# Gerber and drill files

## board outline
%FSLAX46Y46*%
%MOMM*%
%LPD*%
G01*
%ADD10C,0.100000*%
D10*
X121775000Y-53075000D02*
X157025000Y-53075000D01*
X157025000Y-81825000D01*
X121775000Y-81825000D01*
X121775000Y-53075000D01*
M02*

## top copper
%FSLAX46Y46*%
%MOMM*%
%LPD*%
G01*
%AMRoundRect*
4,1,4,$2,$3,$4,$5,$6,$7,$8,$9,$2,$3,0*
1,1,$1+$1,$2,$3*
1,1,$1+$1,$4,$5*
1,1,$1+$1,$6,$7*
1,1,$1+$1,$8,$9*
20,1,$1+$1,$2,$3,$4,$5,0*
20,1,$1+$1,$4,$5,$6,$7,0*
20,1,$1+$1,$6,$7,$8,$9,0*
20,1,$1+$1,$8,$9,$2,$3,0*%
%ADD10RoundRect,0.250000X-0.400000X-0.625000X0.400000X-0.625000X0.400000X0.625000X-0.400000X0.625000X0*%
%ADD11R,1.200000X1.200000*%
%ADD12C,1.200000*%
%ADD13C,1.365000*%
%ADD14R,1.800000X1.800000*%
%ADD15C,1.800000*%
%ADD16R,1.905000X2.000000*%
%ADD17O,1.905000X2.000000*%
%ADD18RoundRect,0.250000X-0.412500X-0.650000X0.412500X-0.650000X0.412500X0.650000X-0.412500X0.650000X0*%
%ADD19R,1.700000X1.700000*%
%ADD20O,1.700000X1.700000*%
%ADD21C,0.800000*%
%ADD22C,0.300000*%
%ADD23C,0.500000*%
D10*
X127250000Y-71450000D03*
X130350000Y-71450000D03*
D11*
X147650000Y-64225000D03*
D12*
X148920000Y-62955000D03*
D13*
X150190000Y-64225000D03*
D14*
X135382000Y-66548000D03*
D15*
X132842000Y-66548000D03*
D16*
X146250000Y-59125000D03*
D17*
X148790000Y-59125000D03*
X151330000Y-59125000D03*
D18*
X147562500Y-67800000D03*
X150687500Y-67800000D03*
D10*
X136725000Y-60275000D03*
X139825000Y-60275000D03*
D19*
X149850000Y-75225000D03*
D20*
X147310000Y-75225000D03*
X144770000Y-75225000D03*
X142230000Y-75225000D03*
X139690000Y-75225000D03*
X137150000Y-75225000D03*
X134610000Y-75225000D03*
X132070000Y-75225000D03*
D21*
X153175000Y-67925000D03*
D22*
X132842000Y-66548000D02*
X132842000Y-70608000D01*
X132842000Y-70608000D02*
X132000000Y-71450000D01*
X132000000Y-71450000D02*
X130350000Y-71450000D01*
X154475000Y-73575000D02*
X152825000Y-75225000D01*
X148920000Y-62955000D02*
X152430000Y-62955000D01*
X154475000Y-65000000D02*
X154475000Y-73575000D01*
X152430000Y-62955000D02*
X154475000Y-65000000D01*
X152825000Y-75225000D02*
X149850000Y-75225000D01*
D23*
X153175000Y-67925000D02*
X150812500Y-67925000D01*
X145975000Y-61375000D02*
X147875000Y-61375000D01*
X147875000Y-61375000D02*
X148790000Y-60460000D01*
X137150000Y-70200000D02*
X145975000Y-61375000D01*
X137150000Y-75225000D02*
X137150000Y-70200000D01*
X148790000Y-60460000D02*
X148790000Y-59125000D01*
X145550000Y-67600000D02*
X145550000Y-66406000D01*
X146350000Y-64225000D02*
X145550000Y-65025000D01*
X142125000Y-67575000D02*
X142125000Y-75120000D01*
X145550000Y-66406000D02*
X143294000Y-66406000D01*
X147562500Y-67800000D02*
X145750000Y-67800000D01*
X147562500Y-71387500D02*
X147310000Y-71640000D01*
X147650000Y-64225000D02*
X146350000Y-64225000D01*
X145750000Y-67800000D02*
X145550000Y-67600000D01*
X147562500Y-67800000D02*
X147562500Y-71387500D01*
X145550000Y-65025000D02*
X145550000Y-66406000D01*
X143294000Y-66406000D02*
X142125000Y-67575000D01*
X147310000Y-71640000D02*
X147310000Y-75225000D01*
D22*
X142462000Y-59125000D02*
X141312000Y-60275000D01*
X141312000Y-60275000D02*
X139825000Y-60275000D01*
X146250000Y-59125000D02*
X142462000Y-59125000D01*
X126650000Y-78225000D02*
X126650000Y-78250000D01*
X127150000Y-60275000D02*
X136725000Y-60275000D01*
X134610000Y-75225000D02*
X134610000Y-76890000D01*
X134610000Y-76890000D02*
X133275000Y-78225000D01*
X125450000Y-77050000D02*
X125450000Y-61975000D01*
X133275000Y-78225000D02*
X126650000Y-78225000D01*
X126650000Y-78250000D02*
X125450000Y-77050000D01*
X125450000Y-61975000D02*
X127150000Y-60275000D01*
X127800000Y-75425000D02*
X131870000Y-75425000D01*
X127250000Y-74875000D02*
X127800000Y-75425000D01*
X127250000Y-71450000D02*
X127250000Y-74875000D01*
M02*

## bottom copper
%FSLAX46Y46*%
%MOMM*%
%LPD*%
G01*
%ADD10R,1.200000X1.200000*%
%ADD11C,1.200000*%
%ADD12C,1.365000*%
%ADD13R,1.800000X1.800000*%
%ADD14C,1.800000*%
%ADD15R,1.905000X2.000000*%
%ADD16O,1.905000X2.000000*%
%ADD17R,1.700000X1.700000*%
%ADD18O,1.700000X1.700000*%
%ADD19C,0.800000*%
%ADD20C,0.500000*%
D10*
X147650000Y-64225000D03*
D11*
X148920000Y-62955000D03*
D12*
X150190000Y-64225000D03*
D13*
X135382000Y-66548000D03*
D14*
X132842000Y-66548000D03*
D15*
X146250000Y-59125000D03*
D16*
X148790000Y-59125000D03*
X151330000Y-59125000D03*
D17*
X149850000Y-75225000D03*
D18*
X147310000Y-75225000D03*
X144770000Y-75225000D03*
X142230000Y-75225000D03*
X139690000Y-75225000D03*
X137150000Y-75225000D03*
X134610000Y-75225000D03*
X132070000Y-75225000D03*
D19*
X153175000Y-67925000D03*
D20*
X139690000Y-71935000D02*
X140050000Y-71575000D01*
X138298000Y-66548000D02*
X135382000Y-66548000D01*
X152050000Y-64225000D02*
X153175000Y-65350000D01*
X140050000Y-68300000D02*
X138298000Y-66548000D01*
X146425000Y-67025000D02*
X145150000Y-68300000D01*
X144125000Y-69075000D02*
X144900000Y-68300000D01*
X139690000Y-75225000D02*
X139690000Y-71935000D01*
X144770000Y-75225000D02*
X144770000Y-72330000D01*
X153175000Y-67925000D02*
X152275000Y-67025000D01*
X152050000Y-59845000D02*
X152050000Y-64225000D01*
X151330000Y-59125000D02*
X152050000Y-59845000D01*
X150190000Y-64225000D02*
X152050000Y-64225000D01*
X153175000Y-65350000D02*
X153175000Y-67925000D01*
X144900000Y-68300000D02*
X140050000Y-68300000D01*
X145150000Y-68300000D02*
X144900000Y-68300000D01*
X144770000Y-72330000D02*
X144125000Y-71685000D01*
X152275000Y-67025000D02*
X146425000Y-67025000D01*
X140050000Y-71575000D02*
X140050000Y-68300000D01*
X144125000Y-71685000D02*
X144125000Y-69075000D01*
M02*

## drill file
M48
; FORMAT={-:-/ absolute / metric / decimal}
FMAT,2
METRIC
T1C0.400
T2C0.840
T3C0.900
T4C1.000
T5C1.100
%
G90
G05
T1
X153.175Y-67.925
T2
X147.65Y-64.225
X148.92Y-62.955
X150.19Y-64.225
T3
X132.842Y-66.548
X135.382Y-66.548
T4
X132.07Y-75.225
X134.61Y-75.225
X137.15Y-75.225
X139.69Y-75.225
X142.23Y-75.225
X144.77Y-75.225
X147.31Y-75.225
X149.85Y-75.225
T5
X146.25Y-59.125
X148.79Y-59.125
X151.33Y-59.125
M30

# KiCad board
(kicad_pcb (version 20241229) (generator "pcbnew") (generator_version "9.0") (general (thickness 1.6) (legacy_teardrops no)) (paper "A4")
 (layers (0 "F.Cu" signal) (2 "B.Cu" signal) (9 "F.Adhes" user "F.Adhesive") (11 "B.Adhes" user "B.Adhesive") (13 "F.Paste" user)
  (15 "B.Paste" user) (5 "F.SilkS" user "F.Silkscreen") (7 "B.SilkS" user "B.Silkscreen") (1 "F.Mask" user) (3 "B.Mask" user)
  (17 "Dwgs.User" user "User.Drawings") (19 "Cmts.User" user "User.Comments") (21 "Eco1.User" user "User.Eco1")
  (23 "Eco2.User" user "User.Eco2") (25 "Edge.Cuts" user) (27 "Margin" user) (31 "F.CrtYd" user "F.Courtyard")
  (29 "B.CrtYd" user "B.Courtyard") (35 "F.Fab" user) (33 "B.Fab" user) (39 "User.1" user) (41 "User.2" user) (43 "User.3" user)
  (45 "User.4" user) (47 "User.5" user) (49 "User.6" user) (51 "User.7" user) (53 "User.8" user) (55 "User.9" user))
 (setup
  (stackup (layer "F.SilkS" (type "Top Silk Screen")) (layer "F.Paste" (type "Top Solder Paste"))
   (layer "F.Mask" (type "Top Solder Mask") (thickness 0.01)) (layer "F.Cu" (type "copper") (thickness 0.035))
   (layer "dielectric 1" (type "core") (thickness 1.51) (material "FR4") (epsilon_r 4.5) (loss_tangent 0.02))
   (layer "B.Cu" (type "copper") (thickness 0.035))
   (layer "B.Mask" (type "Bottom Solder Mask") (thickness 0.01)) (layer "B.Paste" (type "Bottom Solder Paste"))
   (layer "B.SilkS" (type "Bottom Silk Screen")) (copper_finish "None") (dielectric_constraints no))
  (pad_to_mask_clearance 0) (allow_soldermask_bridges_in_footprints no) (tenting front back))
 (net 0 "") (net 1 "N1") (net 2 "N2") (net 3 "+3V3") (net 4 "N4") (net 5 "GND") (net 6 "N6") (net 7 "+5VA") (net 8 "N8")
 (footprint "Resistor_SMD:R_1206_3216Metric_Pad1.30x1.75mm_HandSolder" (layer "F.Cu") (at 128.8 71.45)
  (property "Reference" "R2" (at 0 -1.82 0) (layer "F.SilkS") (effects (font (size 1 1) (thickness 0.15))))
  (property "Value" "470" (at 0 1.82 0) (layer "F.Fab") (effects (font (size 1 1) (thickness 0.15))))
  (pad "1" smd roundrect (at -1.55 0) (size 1.3 1.75) (layers "F.Cu" "F.Mask" "F.Paste") (roundrect_rratio 0.192308) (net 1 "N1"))
  (pad "2" smd roundrect (at 1.55 0) (size 1.3 1.75) (layers "F.Cu" "F.Mask" "F.Paste") (roundrect_rratio 0.192308) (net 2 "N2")))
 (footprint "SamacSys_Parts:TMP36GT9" (layer "F.Cu") (at 147.65 64.225 90)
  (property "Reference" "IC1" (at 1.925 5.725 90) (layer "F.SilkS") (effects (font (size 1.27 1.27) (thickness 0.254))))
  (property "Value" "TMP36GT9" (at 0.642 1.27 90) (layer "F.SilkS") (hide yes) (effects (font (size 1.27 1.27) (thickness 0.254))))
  (pad "1" thru_hole rect (at 0 0 90) (size 1.2 1.2) (drill 0.84) (layers "*.Cu" "*.Mask") (remove_unused_layers no) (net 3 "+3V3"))
  (pad "2" thru_hole circle (at 1.27 1.27 90) (size 1.2 1.2) (drill 0.84) (layers "*.Cu" "*.Mask") (remove_unused_layers no) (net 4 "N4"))
  (pad "3" thru_hole circle (at 0 2.54 90) (size 1.365 1.365) (drill 0.84) (layers "*.Cu" "*.Mask") (remove_unused_layers no) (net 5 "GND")))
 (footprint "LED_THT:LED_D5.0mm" (layer "F.Cu") (at 135.382 66.548 180)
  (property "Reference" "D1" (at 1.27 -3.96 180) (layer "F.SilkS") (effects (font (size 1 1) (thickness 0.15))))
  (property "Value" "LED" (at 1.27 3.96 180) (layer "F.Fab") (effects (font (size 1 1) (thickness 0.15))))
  (pad "1" thru_hole rect (at 0 0 180) (size 1.8 1.8) (drill 0.9) (layers "*.Cu" "*.Mask") (remove_unused_layers no) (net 5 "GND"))
  (pad "2" thru_hole circle (at 2.54 0 180) (size 1.8 1.8) (drill 0.9) (layers "*.Cu" "*.Mask") (remove_unused_layers no) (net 2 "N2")))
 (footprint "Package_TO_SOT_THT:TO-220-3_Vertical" (layer "F.Cu") (at 146.25 59.125)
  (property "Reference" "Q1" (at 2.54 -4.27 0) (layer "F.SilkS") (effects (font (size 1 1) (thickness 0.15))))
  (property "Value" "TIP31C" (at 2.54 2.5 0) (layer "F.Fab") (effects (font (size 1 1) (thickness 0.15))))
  (pad "1" thru_hole rect (at 0 0) (size 1.905 2) (drill 1.1) (layers "*.Cu" "*.Mask") (remove_unused_layers no) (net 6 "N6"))
  (pad "2" thru_hole oval (at 2.54 0) (size 1.905 2) (drill 1.1) (layers "*.Cu" "*.Mask") (remove_unused_layers no) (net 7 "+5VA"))
  (pad "3" thru_hole oval (at 5.08 0) (size 1.905 2) (drill 1.1) (layers "*.Cu" "*.Mask") (remove_unused_layers no) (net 5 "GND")))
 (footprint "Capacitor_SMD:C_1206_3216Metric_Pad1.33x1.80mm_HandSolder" (layer "F.Cu") (at 149.125 67.8)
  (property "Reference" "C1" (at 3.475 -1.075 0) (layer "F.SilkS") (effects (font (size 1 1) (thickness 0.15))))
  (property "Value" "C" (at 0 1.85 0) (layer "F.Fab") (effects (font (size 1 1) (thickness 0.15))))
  (pad "1" smd roundrect (at -1.5625 0) (size 1.325 1.8) (layers "F.Cu" "F.Mask" "F.Paste") (roundrect_rratio 0.188679) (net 3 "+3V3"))
  (pad "2" smd roundrect (at 1.5625 0) (size 1.325 1.8) (layers "F.Cu" "F.Mask" "F.Paste") (roundrect_rratio 0.188679) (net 5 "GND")))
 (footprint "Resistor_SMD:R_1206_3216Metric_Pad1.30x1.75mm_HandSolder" (layer "F.Cu") (at 138.275 60.275)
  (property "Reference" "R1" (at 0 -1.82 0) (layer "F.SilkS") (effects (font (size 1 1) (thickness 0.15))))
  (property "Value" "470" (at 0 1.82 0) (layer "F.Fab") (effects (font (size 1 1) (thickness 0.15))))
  (pad "1" smd roundrect (at -1.55 0) (size 1.3 1.75) (layers "F.Cu" "F.Mask" "F.Paste") (roundrect_rratio 0.192308) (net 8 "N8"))
  (pad "2" smd roundrect (at 1.55 0) (size 1.3 1.75) (layers "F.Cu" "F.Mask" "F.Paste") (roundrect_rratio 0.192308) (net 6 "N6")))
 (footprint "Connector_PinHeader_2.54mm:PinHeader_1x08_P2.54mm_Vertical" (layer "F.Cu") (at 149.85 75.225 -90)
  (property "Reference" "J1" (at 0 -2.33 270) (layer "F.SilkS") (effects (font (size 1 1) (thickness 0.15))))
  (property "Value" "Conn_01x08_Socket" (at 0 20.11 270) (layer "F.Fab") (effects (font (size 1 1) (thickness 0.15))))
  (pad "1" thru_hole rect (at 0 0 270) (size 1.7 1.7) (drill 1) (layers "*.Cu" "*.Mask") (remove_unused_layers no) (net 4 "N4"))
  (pad "2" thru_hole oval (at 0 2.54 270) (size 1.7 1.7) (drill 1) (layers "*.Cu" "*.Mask") (remove_unused_layers no) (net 3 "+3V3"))
  (pad "3" thru_hole oval (at 0 5.08 270) (size 1.7 1.7) (drill 1) (layers "*.Cu" "*.Mask") (remove_unused_layers no) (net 5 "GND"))
  (pad "4" thru_hole oval (at 0 7.62 270) (size 1.7 1.7) (drill 1) (layers "*.Cu" "*.Mask") (remove_unused_layers no) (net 3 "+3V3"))
  (pad "5" thru_hole oval (at 0 10.16 270) (size 1.7 1.7) (drill 1) (layers "*.Cu" "*.Mask") (remove_unused_layers no) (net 5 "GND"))
  (pad "6" thru_hole oval (at 0 12.7 270) (size 1.7 1.7) (drill 1) (layers "*.Cu" "*.Mask") (remove_unused_layers no) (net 7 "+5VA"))
  (pad "7" thru_hole oval (at 0 15.24 270) (size 1.7 1.7) (drill 1) (layers "*.Cu" "*.Mask") (remove_unused_layers no) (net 8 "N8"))
  (pad "8" thru_hole oval (at 0 17.78 270) (size 1.7 1.7) (drill 1) (layers "*.Cu" "*.Mask") (remove_unused_layers no) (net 1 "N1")))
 (gr_rect (start 121.775 53.075) (end 157.025 81.825) (stroke (width 0.1) (type solid)) (fill no) (layer "Edge.Cuts"))
 (segment (start 132.842 66.548) (end 132.842 70.608) (width 0.3) (layer "F.Cu") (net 2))
 (segment (start 132.842 70.608) (end 132 71.45) (width 0.3) (layer "F.Cu") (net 2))
 (segment (start 132 71.45) (end 130.35 71.45) (width 0.3) (layer "F.Cu") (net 2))
 (segment (start 154.475 73.575) (end 152.825 75.225) (width 0.3) (layer "F.Cu") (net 4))
 (segment (start 148.92 62.955) (end 152.43 62.955) (width 0.3) (layer "F.Cu") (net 4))
 (segment (start 154.475 65) (end 154.475 73.575) (width 0.3) (layer "F.Cu") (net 4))
 (segment (start 152.43 62.955) (end 154.475 65) (width 0.3) (layer "F.Cu") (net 4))
 (segment (start 152.825 75.225) (end 149.85 75.225) (width 0.3) (layer "F.Cu") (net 4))
 (segment (start 153.175 67.925) (end 150.8125 67.925) (width 0.5) (layer "F.Cu") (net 5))
 (via (at 153.175 67.925) (size 0.8) (drill 0.4) (layers "F.Cu" "B.Cu") (free yes) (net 5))
 (segment (start 139.69 71.935) (end 140.05 71.575) (width 0.5) (layer "B.Cu") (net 5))
 (segment (start 138.298 66.548) (end 135.382 66.548) (width 0.5) (layer "B.Cu") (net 5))
 (segment (start 152.05 64.225) (end 153.175 65.35) (width 0.5) (layer "B.Cu") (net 5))
 (segment (start 140.05 68.3) (end 138.298 66.548) (width 0.5) (layer "B.Cu") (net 5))
 (segment (start 146.425 67.025) (end 145.15 68.3) (width 0.5) (layer "B.Cu") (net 5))
 (segment (start 144.125 69.075) (end 144.9 68.3) (width 0.5) (layer "B.Cu") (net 5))
 (segment (start 139.69 75.225) (end 139.69 71.935) (width 0.5) (layer "B.Cu") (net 5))
 (segment (start 144.77 75.225) (end 144.77 72.33) (width 0.5) (layer "B.Cu") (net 5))
 (segment (start 153.175 67.925) (end 152.275 67.025) (width 0.5) (layer "B.Cu") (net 5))
 (segment (start 152.05 59.845) (end 152.05 64.225) (width 0.5) (layer "B.Cu") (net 5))
 (segment (start 151.33 59.125) (end 152.05 59.845) (width 0.5) (layer "B.Cu") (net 5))
 (segment (start 150.19 64.225) (end 152.05 64.225) (width 0.5) (layer "B.Cu") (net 5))
 (segment (start 153.175 65.35) (end 153.175 67.925) (width 0.5) (layer "B.Cu") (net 5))
 (segment (start 144.9 68.3) (end 140.05 68.3) (width 0.5) (layer "B.Cu") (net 5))
 (segment (start 145.15 68.3) (end 144.9 68.3) (width 0.5) (layer "B.Cu") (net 5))
 (segment (start 144.77 72.33) (end 144.125 71.685) (width 0.5) (layer "B.Cu") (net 5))
 (segment (start 152.275 67.025) (end 146.425 67.025) (width 0.5) (layer "B.Cu") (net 5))
 (segment (start 140.05 71.575) (end 140.05 68.3) (width 0.5) (layer "B.Cu") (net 5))
 (segment (start 144.125 71.685) (end 144.125 69.075) (width 0.5) (layer "B.Cu") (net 5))
 (segment (start 145.975 61.375) (end 147.875 61.375) (width 0.5) (layer "F.Cu") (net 7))
 (segment (start 147.875 61.375) (end 148.79 60.46) (width 0.5) (layer "F.Cu") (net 7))
 (segment (start 137.15 70.2) (end 145.975 61.375) (width 0.5) (layer "F.Cu") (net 7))
 (segment (start 137.15 75.225) (end 137.15 70.2) (width 0.5) (layer "F.Cu") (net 7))
 (segment (start 148.79 60.46) (end 148.79 59.125) (width 0.5) (layer "F.Cu") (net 7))
 (segment (start 145.55 67.6) (end 145.55 66.406) (width 0.5) (layer "F.Cu") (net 3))
 (segment (start 146.35 64.225) (end 145.55 65.025) (width 0.5) (layer "F.Cu") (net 3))
 (segment (start 142.125 67.575) (end 142.125 75.12) (width 0.5) (layer "F.Cu") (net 3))
 (segment (start 145.55 66.406) (end 143.294 66.406) (width 0.5) (layer "F.Cu") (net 3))
 (segment (start 147.5625 67.8) (end 145.75 67.8) (width 0.5) (layer "F.Cu") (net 3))
 (segment (start 147.5625 71.3875) (end 147.31 71.64) (width 0.5) (layer "F.Cu") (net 3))
 (segment (start 147.65 64.225) (end 146.35 64.225) (width 0.5) (layer "F.Cu") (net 3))
 (segment (start 145.75 67.8) (end 145.55 67.6) (width 0.5) (layer "F.Cu") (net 3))
 (segment (start 147.5625 67.8) (end 147.5625 71.3875) (width 0.5) (layer "F.Cu") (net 3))
 (segment (start 145.55 65.025) (end 145.55 66.406) (width 0.5) (layer "F.Cu") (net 3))
 (segment (start 143.294 66.406) (end 142.125 67.575) (width 0.5) (layer "F.Cu") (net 3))
 (segment (start 147.31 71.64) (end 147.31 75.225) (width 0.5) (layer "F.Cu") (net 3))
 (segment (start 142.462 59.125) (end 141.312 60.275) (width 0.3) (layer "F.Cu") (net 6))
 (segment (start 141.312 60.275) (end 139.825 60.275) (width 0.3) (layer "F.Cu") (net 6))
 (segment (start 146.25 59.125) (end 142.462 59.125) (width 0.3) (layer "F.Cu") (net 6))
 (segment (start 126.65 78.225) (end 126.65 78.25) (width 0.3) (layer "F.Cu") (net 8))
 (segment (start 127.15 60.275) (end 136.725 60.275) (width 0.3) (layer "F.Cu") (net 8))
 (segment (start 134.61 75.225) (end 134.61 76.89) (width 0.3) (layer "F.Cu") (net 8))
 (segment (start 134.61 76.89) (end 133.275 78.225) (width 0.3) (layer "F.Cu") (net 8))
 (segment (start 125.45 77.05) (end 125.45 61.975) (width 0.3) (layer "F.Cu") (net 8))
 (segment (start 133.275 78.225) (end 126.65 78.225) (width 0.3) (layer "F.Cu") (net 8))
 (segment (start 126.65 78.25) (end 125.45 77.05) (width 0.3) (layer "F.Cu") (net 8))
 (segment (start 125.45 61.975) (end 127.15 60.275) (width 0.3) (layer "F.Cu") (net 8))
 (segment (start 127.8 75.425) (end 131.87 75.425) (width 0.3) (layer "F.Cu") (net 1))
 (segment (start 127.25 74.875) (end 127.8 75.425) (width 0.3) (layer "F.Cu") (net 1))
 (segment (start 127.25 71.45) (end 127.25 74.875) (width 0.3) (layer "F.Cu") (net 1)))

